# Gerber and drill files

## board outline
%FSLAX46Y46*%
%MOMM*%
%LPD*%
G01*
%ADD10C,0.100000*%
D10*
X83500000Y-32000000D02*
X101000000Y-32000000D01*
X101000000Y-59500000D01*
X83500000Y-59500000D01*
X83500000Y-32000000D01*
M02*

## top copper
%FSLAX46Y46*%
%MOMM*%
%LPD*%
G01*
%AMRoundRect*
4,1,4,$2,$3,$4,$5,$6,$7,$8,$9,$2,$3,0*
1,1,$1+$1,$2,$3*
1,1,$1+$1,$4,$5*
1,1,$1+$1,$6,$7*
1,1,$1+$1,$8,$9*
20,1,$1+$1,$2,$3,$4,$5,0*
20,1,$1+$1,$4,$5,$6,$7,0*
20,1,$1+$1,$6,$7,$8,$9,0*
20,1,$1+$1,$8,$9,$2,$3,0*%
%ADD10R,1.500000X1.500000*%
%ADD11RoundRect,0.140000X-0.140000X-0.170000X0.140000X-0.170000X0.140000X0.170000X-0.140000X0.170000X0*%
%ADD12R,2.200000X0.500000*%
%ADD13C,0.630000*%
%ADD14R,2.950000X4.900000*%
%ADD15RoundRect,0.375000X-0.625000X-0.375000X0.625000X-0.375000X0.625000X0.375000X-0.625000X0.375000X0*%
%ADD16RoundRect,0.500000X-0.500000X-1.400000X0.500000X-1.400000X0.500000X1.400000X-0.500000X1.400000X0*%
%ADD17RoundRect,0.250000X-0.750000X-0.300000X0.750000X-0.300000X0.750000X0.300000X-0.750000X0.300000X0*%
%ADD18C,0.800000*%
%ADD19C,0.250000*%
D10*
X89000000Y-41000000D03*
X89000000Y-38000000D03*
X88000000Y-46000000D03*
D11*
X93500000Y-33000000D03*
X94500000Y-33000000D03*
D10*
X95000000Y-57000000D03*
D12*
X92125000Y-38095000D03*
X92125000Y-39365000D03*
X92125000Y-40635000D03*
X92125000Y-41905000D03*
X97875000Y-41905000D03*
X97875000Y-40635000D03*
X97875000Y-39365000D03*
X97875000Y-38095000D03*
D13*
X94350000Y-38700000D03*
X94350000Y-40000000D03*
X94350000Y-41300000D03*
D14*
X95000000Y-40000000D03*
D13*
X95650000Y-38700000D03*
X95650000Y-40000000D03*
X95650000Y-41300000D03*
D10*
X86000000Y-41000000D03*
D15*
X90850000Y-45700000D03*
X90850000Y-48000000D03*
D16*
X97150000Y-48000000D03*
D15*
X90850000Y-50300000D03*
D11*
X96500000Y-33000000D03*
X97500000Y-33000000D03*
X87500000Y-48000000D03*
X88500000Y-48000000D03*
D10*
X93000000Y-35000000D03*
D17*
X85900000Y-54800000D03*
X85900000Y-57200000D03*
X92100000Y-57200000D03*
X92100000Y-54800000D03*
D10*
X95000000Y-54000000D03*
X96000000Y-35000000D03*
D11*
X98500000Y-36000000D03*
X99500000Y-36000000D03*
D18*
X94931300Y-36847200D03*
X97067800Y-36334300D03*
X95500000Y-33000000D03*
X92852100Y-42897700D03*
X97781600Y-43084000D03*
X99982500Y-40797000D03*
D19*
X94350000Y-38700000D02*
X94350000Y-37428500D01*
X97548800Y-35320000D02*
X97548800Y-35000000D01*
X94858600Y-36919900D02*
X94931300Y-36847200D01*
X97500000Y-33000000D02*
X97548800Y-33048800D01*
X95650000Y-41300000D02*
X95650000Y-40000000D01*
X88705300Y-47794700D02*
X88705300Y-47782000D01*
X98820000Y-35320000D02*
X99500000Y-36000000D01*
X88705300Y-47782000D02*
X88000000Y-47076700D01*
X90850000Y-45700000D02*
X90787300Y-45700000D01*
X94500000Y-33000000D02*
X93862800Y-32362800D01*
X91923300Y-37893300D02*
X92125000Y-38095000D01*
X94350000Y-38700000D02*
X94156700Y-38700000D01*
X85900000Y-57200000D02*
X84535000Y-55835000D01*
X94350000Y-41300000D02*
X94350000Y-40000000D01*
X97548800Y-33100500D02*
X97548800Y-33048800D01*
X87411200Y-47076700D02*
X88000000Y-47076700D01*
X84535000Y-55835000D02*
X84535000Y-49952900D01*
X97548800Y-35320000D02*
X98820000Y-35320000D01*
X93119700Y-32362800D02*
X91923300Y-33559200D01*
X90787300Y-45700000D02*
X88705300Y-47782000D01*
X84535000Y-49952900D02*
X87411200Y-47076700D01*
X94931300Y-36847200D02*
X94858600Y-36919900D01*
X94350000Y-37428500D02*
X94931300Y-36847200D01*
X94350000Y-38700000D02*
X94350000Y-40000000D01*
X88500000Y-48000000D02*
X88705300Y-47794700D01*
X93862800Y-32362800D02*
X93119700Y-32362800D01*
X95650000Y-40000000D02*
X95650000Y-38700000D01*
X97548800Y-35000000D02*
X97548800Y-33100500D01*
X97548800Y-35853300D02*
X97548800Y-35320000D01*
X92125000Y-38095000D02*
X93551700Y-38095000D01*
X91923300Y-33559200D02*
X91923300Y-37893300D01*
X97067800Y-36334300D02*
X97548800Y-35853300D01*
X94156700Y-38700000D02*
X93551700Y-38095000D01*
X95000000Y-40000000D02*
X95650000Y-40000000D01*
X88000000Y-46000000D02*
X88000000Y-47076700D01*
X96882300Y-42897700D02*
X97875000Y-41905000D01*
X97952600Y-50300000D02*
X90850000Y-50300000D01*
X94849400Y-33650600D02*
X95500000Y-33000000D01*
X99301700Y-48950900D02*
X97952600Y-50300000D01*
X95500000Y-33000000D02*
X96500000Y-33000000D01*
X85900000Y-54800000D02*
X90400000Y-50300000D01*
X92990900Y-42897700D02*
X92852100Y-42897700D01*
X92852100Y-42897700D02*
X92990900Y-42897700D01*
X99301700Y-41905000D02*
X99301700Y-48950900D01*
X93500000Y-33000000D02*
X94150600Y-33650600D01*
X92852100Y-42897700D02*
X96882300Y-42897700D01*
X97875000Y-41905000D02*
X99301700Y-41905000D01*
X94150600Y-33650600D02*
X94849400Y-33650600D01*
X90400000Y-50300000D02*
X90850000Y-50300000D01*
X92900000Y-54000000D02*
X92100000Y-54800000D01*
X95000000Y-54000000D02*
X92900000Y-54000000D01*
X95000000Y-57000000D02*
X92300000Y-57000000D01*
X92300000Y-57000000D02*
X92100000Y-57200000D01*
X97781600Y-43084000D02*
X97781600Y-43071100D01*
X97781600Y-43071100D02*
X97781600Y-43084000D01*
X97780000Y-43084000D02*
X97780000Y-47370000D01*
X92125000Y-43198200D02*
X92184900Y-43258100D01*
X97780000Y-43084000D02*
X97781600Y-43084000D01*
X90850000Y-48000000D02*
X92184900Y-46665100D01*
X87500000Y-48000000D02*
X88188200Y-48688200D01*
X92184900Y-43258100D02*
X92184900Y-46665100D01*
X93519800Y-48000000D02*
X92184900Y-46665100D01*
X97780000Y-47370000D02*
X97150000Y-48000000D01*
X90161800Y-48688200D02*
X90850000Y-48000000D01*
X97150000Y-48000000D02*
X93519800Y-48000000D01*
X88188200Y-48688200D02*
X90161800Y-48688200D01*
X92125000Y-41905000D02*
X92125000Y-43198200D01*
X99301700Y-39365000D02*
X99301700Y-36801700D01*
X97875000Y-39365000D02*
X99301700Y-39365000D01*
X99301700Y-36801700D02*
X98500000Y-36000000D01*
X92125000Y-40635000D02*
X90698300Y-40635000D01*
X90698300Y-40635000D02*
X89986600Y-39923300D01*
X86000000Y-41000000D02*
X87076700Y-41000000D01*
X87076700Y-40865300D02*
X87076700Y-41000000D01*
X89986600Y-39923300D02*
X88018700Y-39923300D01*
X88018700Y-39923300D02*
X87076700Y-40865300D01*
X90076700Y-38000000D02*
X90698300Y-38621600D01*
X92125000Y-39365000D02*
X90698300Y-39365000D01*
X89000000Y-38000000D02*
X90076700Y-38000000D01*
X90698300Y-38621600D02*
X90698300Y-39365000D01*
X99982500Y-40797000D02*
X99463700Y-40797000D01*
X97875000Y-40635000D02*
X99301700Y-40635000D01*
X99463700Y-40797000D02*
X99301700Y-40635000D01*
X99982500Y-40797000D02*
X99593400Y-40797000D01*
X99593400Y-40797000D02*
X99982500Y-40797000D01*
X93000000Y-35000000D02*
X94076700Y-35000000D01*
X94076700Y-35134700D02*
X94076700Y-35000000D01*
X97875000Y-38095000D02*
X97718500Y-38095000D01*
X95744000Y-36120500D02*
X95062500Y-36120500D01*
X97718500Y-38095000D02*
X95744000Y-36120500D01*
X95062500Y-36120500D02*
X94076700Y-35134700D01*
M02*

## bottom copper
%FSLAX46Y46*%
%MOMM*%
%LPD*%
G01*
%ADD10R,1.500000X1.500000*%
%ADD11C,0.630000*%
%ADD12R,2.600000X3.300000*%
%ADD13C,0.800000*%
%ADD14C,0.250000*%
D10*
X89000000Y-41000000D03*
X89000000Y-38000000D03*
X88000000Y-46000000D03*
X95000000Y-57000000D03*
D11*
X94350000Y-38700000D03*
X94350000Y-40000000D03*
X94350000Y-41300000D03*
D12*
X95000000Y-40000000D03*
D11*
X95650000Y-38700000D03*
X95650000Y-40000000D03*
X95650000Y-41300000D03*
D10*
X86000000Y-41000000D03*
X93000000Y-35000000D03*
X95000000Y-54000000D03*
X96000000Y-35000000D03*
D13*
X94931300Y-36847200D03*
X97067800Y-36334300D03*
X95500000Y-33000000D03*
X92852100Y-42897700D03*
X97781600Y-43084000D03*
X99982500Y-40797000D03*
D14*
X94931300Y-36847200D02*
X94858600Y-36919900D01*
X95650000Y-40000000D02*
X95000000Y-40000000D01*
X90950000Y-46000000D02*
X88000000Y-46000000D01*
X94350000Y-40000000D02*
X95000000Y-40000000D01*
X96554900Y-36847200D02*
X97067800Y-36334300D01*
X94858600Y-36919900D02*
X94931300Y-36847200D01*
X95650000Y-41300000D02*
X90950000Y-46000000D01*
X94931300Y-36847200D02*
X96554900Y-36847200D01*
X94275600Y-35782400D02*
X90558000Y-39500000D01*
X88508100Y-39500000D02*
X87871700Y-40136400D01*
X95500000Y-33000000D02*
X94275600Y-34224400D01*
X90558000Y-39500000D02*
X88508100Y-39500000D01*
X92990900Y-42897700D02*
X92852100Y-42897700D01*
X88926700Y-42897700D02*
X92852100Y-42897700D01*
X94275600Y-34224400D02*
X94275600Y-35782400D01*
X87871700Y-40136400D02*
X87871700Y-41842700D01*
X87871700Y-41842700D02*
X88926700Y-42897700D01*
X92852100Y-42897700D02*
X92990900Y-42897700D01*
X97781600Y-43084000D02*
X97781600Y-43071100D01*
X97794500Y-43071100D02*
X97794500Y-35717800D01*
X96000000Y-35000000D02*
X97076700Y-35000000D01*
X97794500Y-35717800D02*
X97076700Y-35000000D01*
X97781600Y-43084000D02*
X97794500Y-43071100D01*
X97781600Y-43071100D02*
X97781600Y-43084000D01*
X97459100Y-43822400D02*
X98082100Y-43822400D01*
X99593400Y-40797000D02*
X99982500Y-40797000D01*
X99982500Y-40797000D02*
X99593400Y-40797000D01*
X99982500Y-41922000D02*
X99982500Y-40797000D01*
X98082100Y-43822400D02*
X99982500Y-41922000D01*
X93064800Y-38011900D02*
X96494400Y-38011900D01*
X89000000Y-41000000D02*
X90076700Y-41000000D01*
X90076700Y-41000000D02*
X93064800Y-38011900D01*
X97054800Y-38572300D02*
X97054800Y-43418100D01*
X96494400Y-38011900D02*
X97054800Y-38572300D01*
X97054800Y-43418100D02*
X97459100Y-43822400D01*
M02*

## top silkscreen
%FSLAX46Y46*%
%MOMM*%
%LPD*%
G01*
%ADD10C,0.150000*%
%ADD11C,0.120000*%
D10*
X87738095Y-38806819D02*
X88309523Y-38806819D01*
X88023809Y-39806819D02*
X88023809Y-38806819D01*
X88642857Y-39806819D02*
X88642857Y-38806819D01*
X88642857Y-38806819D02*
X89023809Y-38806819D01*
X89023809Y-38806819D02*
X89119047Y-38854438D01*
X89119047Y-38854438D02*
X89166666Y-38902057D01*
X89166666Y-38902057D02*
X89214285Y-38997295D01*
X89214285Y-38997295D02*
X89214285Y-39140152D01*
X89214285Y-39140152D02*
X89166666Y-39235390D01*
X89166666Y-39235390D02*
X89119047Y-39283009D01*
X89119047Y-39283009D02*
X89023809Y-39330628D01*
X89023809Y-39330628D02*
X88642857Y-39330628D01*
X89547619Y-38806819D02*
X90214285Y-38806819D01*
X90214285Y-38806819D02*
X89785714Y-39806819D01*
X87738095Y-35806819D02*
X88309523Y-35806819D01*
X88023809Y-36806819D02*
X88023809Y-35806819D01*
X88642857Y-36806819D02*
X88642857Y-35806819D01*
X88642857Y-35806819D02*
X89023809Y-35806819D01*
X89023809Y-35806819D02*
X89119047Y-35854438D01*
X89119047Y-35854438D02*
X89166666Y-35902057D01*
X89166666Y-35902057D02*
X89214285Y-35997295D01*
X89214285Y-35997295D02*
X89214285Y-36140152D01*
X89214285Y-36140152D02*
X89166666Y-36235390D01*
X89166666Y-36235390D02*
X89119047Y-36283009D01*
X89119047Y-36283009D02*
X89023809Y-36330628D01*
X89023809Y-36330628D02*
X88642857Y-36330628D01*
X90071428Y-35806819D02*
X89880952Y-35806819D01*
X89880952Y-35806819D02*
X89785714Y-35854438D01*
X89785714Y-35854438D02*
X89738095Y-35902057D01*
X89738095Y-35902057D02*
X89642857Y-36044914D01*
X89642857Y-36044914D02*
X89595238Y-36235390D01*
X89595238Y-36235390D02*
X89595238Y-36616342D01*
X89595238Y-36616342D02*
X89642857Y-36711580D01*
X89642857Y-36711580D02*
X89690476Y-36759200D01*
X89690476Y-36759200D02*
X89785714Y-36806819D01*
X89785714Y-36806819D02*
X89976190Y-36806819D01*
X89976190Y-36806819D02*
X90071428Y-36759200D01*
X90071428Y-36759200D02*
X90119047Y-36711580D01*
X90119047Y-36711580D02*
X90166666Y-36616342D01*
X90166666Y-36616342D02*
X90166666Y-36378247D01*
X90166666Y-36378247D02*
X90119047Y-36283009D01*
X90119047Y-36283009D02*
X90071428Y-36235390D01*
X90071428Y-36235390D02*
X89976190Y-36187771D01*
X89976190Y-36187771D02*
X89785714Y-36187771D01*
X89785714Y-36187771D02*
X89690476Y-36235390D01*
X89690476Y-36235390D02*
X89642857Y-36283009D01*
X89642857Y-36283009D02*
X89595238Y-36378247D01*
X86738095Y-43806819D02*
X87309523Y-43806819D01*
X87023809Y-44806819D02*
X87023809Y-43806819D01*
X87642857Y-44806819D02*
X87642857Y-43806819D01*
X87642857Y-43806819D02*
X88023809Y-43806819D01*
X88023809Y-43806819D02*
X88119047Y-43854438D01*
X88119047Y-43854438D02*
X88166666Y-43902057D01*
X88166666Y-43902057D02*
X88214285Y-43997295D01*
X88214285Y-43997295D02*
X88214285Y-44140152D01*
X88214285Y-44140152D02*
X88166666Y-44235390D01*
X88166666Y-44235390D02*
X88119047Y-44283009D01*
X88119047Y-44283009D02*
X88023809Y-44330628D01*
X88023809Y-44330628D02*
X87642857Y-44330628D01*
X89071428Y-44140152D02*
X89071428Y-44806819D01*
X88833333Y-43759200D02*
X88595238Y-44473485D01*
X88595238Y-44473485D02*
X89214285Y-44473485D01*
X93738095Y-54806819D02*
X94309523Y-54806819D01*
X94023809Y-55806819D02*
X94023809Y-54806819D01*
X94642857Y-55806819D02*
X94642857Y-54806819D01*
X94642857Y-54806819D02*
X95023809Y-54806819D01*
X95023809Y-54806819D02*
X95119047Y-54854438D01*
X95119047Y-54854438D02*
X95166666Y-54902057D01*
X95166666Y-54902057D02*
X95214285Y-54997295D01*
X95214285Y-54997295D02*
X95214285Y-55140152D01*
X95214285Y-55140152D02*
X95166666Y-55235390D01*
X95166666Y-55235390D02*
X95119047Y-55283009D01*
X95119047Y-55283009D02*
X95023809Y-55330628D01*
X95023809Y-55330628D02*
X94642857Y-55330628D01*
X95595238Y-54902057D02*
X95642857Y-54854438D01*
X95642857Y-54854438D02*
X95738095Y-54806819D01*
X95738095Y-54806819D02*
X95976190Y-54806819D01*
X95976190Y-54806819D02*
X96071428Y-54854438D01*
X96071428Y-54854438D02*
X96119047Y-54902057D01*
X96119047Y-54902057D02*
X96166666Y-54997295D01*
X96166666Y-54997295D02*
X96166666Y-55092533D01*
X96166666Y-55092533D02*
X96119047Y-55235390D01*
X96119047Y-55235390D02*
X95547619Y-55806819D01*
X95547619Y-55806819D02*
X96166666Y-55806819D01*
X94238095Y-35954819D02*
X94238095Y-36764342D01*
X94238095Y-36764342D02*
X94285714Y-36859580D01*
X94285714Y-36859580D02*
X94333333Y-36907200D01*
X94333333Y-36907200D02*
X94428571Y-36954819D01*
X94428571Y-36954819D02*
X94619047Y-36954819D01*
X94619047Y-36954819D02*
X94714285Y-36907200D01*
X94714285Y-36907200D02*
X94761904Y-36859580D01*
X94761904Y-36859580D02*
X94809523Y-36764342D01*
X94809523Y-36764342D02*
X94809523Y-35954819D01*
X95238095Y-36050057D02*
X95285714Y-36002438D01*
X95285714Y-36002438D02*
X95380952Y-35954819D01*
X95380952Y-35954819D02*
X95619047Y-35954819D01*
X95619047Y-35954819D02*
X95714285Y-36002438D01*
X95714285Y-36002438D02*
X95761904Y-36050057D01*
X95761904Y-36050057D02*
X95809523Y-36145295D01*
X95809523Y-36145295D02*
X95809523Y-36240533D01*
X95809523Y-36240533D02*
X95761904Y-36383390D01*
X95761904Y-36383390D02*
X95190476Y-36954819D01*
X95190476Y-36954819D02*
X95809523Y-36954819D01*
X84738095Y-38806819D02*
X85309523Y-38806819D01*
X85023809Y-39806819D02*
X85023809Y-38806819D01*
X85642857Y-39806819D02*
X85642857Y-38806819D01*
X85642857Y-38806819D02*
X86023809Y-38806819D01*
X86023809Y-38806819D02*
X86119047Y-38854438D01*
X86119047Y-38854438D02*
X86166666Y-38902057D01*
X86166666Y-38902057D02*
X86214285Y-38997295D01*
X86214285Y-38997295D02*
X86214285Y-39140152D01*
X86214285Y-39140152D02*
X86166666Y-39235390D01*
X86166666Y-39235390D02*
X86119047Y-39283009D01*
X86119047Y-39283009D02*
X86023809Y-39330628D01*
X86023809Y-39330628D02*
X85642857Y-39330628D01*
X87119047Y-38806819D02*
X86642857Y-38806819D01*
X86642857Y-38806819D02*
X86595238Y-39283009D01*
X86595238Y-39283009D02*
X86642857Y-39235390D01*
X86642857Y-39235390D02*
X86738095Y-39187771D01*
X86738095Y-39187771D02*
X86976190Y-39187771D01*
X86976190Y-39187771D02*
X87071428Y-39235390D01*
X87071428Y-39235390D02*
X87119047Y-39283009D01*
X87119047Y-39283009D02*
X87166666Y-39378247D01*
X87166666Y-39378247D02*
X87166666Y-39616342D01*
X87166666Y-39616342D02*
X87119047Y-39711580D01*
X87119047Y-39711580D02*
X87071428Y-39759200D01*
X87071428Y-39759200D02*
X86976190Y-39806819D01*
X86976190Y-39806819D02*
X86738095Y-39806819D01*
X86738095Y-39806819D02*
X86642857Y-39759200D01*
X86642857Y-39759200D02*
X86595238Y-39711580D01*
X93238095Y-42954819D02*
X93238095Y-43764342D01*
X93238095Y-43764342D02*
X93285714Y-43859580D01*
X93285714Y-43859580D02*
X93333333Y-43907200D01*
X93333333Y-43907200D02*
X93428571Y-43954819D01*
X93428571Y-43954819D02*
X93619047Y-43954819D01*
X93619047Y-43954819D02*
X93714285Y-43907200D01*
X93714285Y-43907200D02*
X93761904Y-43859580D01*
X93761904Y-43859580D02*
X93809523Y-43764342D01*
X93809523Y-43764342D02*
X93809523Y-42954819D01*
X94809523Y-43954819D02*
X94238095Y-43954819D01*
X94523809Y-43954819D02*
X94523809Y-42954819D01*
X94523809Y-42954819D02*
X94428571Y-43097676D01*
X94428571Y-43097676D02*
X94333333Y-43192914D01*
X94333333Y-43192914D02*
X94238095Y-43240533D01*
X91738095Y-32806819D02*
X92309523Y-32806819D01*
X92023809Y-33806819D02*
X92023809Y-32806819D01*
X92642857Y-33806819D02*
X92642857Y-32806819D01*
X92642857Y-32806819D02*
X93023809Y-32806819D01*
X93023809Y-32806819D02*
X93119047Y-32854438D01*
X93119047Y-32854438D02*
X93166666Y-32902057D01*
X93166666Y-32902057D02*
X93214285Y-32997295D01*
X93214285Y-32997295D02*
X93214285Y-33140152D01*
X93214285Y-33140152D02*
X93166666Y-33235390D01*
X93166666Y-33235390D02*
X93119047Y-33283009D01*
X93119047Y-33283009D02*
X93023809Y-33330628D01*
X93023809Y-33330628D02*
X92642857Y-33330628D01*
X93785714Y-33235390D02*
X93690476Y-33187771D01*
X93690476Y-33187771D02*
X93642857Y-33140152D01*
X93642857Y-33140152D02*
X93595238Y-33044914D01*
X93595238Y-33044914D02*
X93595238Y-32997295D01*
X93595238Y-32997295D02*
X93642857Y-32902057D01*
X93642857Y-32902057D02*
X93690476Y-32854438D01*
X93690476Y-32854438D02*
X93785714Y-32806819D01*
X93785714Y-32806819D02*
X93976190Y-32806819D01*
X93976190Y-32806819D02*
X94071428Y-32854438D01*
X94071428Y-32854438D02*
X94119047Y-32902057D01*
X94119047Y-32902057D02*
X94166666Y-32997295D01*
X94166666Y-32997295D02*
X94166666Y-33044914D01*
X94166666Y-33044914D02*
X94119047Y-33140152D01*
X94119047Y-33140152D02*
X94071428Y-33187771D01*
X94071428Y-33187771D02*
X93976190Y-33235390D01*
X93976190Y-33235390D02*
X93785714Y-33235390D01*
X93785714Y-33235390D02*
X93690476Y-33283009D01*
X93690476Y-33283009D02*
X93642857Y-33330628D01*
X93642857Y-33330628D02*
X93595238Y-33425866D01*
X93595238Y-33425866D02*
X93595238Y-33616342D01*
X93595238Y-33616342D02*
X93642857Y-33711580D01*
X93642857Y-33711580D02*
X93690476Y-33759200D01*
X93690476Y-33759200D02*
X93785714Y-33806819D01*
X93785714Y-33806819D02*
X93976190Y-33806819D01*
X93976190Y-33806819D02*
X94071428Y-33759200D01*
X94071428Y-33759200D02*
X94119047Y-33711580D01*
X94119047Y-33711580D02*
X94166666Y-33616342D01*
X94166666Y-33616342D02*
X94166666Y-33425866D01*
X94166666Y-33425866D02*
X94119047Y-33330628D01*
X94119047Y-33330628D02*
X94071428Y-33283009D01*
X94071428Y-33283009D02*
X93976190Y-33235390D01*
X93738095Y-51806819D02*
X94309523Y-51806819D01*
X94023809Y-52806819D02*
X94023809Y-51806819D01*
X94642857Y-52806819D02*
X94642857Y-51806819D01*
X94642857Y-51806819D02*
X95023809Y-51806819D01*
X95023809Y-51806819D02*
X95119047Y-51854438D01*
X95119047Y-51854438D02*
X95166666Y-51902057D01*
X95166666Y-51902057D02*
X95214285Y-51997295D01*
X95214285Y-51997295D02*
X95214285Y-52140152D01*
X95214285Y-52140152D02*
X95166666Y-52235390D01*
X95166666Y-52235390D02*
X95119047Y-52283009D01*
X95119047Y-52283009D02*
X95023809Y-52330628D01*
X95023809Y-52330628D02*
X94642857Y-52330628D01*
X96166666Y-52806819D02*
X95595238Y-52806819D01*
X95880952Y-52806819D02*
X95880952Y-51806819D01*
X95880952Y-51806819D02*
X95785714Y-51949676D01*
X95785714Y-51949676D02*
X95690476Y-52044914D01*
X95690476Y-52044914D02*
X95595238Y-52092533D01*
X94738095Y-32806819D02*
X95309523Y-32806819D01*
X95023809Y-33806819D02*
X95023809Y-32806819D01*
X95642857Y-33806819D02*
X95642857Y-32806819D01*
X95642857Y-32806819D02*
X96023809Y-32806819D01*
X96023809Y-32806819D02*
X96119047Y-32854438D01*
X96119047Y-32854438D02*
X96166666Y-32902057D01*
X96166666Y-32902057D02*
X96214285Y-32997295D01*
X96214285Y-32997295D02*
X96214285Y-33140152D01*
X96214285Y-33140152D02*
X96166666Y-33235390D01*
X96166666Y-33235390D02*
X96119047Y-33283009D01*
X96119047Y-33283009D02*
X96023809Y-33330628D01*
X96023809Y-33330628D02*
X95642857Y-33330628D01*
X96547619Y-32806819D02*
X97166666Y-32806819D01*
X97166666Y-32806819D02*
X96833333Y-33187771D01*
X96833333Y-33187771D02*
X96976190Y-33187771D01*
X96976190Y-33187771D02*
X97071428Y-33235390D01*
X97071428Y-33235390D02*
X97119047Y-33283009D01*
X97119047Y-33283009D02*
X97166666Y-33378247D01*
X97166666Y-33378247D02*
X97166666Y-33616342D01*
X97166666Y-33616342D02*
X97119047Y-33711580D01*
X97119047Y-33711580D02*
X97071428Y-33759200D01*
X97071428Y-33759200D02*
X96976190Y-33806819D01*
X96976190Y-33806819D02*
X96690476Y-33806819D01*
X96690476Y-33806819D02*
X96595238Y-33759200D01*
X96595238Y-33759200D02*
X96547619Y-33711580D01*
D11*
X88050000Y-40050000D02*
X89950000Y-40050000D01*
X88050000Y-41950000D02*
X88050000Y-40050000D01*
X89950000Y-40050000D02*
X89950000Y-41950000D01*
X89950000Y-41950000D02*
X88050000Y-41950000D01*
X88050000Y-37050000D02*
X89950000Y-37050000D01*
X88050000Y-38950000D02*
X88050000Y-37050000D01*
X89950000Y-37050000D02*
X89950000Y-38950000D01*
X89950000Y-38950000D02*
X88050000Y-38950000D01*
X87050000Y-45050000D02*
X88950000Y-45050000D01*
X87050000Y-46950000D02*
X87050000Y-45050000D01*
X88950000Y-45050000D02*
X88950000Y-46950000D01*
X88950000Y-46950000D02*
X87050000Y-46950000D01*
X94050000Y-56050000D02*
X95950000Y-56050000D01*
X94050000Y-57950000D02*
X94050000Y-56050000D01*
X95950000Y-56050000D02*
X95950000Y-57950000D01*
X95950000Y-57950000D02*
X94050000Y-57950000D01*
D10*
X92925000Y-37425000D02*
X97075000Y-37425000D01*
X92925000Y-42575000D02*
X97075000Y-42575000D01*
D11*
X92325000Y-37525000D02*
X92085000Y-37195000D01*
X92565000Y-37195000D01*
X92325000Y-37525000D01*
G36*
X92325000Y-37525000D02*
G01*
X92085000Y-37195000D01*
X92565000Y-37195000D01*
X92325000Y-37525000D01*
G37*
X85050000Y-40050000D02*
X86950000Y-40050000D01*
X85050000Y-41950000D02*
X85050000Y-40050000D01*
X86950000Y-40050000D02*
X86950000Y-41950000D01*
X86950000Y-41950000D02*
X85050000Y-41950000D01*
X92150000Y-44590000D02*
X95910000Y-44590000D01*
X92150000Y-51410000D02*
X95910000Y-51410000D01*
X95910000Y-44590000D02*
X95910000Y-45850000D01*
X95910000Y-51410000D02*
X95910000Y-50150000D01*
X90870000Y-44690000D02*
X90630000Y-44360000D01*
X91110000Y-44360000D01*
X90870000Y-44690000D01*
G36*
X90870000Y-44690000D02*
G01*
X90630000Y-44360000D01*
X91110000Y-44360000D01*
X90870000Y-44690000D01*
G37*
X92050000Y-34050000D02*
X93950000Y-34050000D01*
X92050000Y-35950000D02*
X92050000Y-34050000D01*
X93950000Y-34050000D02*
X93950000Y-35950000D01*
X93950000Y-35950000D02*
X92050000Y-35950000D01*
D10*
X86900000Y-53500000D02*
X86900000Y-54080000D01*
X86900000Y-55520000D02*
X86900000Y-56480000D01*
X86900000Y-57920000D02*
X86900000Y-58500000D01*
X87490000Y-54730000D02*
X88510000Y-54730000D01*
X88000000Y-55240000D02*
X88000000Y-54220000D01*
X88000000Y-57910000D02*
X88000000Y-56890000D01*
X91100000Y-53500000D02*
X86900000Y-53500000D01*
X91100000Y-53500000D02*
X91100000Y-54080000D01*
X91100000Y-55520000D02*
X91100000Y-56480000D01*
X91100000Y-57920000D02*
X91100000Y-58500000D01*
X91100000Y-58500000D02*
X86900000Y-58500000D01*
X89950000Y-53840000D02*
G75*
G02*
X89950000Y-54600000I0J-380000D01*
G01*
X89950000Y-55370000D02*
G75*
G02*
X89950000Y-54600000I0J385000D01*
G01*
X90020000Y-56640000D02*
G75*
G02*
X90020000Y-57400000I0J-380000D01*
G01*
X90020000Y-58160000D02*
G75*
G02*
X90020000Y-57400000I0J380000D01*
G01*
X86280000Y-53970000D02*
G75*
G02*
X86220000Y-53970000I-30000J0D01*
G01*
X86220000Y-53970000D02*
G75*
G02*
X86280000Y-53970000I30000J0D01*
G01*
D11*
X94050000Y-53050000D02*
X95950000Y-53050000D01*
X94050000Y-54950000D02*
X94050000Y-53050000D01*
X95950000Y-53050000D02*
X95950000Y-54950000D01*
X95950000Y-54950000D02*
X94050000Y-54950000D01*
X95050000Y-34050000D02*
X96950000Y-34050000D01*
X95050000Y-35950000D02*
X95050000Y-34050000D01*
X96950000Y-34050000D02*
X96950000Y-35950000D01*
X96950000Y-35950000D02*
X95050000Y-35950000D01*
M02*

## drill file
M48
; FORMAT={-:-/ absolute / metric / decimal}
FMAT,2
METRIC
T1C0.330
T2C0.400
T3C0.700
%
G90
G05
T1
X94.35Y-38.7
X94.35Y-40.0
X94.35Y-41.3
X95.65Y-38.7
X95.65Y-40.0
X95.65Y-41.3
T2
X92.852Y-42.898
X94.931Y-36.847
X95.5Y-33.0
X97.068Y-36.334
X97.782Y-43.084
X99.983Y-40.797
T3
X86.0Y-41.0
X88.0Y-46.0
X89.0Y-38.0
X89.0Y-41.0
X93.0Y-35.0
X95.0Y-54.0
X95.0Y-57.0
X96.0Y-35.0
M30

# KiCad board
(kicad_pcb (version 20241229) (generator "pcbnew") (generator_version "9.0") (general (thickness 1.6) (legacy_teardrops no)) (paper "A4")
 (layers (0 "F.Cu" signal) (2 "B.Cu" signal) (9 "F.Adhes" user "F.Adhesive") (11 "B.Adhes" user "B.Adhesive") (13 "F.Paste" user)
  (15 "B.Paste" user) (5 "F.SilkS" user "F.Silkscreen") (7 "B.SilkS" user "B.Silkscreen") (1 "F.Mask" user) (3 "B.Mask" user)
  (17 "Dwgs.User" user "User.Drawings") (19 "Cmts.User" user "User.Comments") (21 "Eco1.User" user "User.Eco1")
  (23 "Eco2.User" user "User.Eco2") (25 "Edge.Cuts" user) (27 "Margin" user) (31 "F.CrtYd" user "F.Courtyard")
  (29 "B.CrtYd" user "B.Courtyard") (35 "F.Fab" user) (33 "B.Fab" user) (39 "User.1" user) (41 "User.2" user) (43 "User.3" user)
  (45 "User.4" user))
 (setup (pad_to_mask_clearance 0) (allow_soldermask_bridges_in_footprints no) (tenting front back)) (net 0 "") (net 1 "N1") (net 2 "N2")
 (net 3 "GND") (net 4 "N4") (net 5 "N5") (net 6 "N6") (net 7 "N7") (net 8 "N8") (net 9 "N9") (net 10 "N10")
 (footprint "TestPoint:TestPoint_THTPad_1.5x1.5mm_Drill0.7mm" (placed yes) (layer "F.Cu") (at 89 41)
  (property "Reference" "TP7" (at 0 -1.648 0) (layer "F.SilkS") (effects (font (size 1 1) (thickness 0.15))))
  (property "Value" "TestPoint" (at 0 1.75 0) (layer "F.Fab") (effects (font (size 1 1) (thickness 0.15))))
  (fp_line (start -0.95 -0.95) (end 0.95 -0.95) (stroke (width 0.12) (type solid)) (layer "F.SilkS"))
  (fp_line (start -0.95 0.95) (end -0.95 -0.95) (stroke (width 0.12) (type solid)) (layer "F.SilkS"))
  (fp_line (start 0.95 -0.95) (end 0.95 0.95) (stroke (width 0.12) (type solid)) (layer "F.SilkS"))
  (fp_line (start 0.95 0.95) (end -0.95 0.95) (stroke (width 0.12) (type solid)) (layer "F.SilkS"))
  (pad "1" thru_hole rect (at 0 0) (size 1.5 1.5) (drill 0.7) (layers "*.Cu" "*.Mask") (remove_unused_layers no) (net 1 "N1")))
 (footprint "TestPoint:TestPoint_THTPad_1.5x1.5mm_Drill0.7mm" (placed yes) (layer "F.Cu") (at 89 38)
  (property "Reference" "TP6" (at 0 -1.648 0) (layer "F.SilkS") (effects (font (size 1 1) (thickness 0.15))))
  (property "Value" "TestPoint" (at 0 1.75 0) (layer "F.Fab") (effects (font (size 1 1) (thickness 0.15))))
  (fp_line (start -0.95 -0.95) (end 0.95 -0.95) (stroke (width 0.12) (type solid)) (layer "F.SilkS"))
  (fp_line (start -0.95 0.95) (end -0.95 -0.95) (stroke (width 0.12) (type solid)) (layer "F.SilkS"))
  (fp_line (start 0.95 -0.95) (end 0.95 0.95) (stroke (width 0.12) (type solid)) (layer "F.SilkS"))
  (fp_line (start 0.95 0.95) (end -0.95 0.95) (stroke (width 0.12) (type solid)) (layer "F.SilkS"))
  (pad "1" thru_hole rect (at 0 0) (size 1.5 1.5) (drill 0.7) (layers "*.Cu" "*.Mask") (remove_unused_layers no) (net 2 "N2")))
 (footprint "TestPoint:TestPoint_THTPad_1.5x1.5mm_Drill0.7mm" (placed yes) (layer "F.Cu") (at 88 46)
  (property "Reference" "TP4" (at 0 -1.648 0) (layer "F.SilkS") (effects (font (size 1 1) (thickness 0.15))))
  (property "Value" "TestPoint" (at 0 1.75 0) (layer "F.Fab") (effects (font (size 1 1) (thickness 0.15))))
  (fp_line (start -0.95 -0.95) (end 0.95 -0.95) (stroke (width 0.12) (type solid)) (layer "F.SilkS"))
  (fp_line (start -0.95 0.95) (end -0.95 -0.95) (stroke (width 0.12) (type solid)) (layer "F.SilkS"))
  (fp_line (start 0.95 -0.95) (end 0.95 0.95) (stroke (width 0.12) (type solid)) (layer "F.SilkS"))
  (fp_line (start 0.95 0.95) (end -0.95 0.95) (stroke (width 0.12) (type solid)) (layer "F.SilkS"))
  (pad "1" thru_hole rect (at 0 0) (size 1.5 1.5) (drill 0.7) (layers "*.Cu" "*.Mask") (remove_unused_layers no) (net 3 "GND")))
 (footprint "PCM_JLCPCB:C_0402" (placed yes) (layer "F.Cu") (at 94 33)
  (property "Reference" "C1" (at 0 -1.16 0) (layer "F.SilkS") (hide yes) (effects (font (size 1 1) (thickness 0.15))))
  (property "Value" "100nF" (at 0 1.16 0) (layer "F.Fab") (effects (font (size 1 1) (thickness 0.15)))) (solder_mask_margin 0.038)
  (pad "1" smd roundrect (at -0.5 0) (size 0.56 0.62) (layers "F.Cu" "F.Mask" "F.Paste") (roundrect_rratio 0.25) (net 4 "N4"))
  (pad "2" smd roundrect (at 0.5 0) (size 0.56 0.62) (layers "F.Cu" "F.Mask" "F.Paste") (roundrect_rratio 0.25) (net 3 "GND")))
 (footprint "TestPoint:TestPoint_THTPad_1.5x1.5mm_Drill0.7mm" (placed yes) (layer "F.Cu") (at 95 57)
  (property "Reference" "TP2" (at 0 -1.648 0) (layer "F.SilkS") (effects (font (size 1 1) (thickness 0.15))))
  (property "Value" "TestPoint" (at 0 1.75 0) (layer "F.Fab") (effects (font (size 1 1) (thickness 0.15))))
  (fp_line (start -0.95 -0.95) (end 0.95 -0.95) (stroke (width 0.12) (type solid)) (layer "F.SilkS"))
  (fp_line (start -0.95 0.95) (end -0.95 -0.95) (stroke (width 0.12) (type solid)) (layer "F.SilkS"))
  (fp_line (start 0.95 -0.95) (end 0.95 0.95) (stroke (width 0.12) (type solid)) (layer "F.SilkS"))
  (fp_line (start 0.95 0.95) (end -0.95 0.95) (stroke (width 0.12) (type solid)) (layer "F.SilkS"))
  (pad "1" thru_hole rect (at 0 0) (size 1.5 1.5) (drill 0.7) (layers "*.Cu" "*.Mask") (remove_unused_layers no) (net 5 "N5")))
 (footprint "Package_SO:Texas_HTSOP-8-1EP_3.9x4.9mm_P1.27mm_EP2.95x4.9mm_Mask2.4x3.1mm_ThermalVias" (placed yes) (layer "F.Cu") (at 95 40)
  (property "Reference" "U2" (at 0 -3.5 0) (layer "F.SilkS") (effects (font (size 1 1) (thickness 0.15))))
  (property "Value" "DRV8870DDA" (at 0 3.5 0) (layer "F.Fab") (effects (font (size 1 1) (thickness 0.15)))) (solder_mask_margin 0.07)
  (fp_line (start -2.075 -2.575) (end 2.075 -2.575) (stroke (width 0.15) (type solid)) (layer "F.SilkS"))
  (fp_line (start -2.075 2.575) (end 2.075 2.575) (stroke (width 0.15) (type solid)) (layer "F.SilkS"))
  (fp_poly
   (pts (xy -2.675 -2.475) (xy -2.915 -2.805) (xy -2.435 -2.805) (xy -2.675 -2.475)) (stroke (width 0.12) (type solid)) (fill yes)
   (layer "F.SilkS"))
  (pad "" smd rect (at 0 0) (size 2.4 3.1) (layers "F.Mask")) (pad "" smd rect (at 0 0) (size 2.4 3.1) (layers "F.Paste"))
  (pad "1" smd rect (at -2.875 -1.905) (size 2.2 0.5) (layers "F.Cu" "F.Mask" "F.Paste") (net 3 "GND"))
  (pad "2" smd rect (at -2.875 -0.635) (size 2.2 0.5) (layers "F.Cu" "F.Mask" "F.Paste") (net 2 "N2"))
  (pad "3" smd rect (at -2.875 0.635) (size 2.2 0.5) (layers "F.Cu" "F.Mask" "F.Paste") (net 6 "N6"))
  (pad "4" smd rect (at -2.875 1.905) (size 2.2 0.5) (layers "F.Cu" "F.Mask" "F.Paste") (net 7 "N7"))
  (pad "5" smd rect (at 2.875 1.905) (size 2.2 0.5) (layers "F.Cu" "F.Mask" "F.Paste") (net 4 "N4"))
  (pad "6" smd rect (at 2.875 0.635) (size 2.2 0.5) (layers "F.Cu" "F.Mask" "F.Paste") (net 1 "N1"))
  (pad "7" smd rect (at 2.875 -0.635) (size 2.2 0.5) (layers "F.Cu" "F.Mask" "F.Paste") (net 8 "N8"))
  (pad "8" smd rect (at 2.875 -1.905) (size 2.2 0.5) (layers "F.Cu" "F.Mask" "F.Paste") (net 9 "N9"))
  (pad "9" thru_hole circle (at -0.65 -1.3) (size 0.63 0.63) (drill 0.33) (layers "*.Cu" "*.Mask") (remove_unused_layers no) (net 3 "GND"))
  (pad "9" thru_hole circle (at -0.65 0) (size 0.63 0.63) (drill 0.33) (layers "*.Cu" "*.Mask") (remove_unused_layers no) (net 3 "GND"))
  (pad "9" thru_hole circle (at -0.65 1.3) (size 0.63 0.63) (drill 0.33) (layers "*.Cu" "*.Mask") (remove_unused_layers no) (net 3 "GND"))
  (pad "9" smd rect (at 0 0) (size 2.6 3.3) (layers "B.Cu") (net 3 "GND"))
  (pad "9" smd rect (at 0 0) (size 2.95 4.9) (layers "F.Cu") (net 3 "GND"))
  (pad "9" thru_hole circle (at 0.65 -1.3) (size 0.63 0.63) (drill 0.33) (layers "*.Cu" "*.Mask") (remove_unused_layers no) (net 3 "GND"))
  (pad "9" thru_hole circle (at 0.65 0) (size 0.63 0.63) (drill 0.33) (layers "*.Cu" "*.Mask") (remove_unused_layers no) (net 3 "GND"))
  (pad "9" thru_hole circle (at 0.65 1.3) (size 0.63 0.63) (drill 0.33) (layers "*.Cu" "*.Mask") (remove_unused_layers no) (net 3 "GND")))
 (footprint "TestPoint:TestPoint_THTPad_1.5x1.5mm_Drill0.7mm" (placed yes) (layer "F.Cu") (at 86 41)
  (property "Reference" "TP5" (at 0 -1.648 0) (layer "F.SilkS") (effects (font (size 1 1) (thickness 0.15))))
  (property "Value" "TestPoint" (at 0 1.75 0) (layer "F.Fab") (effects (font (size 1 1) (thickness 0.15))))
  (fp_line (start -0.95 -0.95) (end 0.95 -0.95) (stroke (width 0.12) (type solid)) (layer "F.SilkS"))
  (fp_line (start -0.95 0.95) (end -0.95 -0.95) (stroke (width 0.12) (type solid)) (layer "F.SilkS"))
  (fp_line (start 0.95 -0.95) (end 0.95 0.95) (stroke (width 0.12) (type solid)) (layer "F.SilkS"))
  (fp_line (start 0.95 0.95) (end -0.95 0.95) (stroke (width 0.12) (type solid)) (layer "F.SilkS"))
  (pad "1" thru_hole rect (at 0 0) (size 1.5 1.5) (drill 0.7) (layers "*.Cu" "*.Mask") (remove_unused_layers no) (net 6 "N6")))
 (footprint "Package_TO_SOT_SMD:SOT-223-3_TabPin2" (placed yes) (layer "F.Cu") (at 94 48)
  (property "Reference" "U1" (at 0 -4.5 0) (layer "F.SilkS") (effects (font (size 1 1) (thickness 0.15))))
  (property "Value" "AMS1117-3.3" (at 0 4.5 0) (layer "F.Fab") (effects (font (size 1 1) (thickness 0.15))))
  (fp_line (start -1.85 -3.41) (end 1.91 -3.41) (stroke (width 0.12) (type solid)) (layer "F.SilkS"))
  (fp_line (start -1.85 3.41) (end 1.91 3.41) (stroke (width 0.12) (type solid)) (layer "F.SilkS"))
  (fp_line (start 1.91 -3.41) (end 1.91 -2.15) (stroke (width 0.12) (type solid)) (layer "F.SilkS"))
  (fp_line (start 1.91 3.41) (end 1.91 2.15) (stroke (width 0.12) (type solid)) (layer "F.SilkS"))
  (fp_poly
   (pts (xy -3.13 -3.31) (xy -3.37 -3.64) (xy -2.89 -3.64) (xy -3.13 -3.31)) (stroke (width 0.12) (type solid)) (fill yes) (layer "F.SilkS"))
  (pad "1" smd roundrect (at -3.15 -2.3) (size 2 1.5) (layers "F.Cu" "F.Mask" "F.Paste") (roundrect_rratio 0.25) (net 3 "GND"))
  (pad "2" smd roundrect (at -3.15 0) (size 2 1.5) (layers "F.Cu" "F.Mask" "F.Paste") (roundrect_rratio 0.25) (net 7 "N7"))
  (pad "2" smd roundrect (at 3.15 0) (size 2 3.8) (layers "F.Cu" "F.Mask" "F.Paste") (roundrect_rratio 0.25) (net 7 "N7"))
  (pad "3" smd roundrect (at -3.15 2.3) (size 2 1.5) (layers "F.Cu" "F.Mask" "F.Paste") (roundrect_rratio 0.25) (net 4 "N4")))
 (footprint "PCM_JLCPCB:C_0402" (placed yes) (layer "F.Cu") (at 97 33)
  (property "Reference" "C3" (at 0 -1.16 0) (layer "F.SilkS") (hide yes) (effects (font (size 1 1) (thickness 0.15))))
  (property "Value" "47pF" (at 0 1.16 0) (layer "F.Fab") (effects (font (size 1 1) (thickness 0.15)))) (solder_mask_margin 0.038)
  (pad "1" smd roundrect (at -0.5 0) (size 0.56 0.62) (layers "F.Cu" "F.Mask" "F.Paste") (roundrect_rratio 0.25) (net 4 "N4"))
  (pad "2" smd roundrect (at 0.5 0) (size 0.56 0.62) (layers "F.Cu" "F.Mask" "F.Paste") (roundrect_rratio 0.25) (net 3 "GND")))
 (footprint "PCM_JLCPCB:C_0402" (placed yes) (layer "F.Cu") (at 88 48)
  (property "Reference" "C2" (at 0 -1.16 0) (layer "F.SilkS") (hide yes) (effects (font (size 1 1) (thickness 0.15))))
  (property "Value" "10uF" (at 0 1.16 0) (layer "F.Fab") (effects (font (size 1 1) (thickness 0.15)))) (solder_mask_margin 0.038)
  (pad "1" smd roundrect (at -0.5 0) (size 0.56 0.62) (layers "F.Cu" "F.Mask" "F.Paste") (roundrect_rratio 0.25) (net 7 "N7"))
  (pad "2" smd roundrect (at 0.5 0) (size 0.56 0.62) (layers "F.Cu" "F.Mask" "F.Paste") (roundrect_rratio 0.25) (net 3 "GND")))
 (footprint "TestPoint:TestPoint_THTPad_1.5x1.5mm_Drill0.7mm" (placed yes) (layer "F.Cu") (at 93 35)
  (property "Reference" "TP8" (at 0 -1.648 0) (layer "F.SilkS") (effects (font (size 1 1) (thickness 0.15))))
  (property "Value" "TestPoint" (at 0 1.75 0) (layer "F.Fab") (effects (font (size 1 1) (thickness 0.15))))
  (fp_line (start -0.95 -0.95) (end 0.95 -0.95) (stroke (width 0.12) (type solid)) (layer "F.SilkS"))
  (fp_line (start -0.95 0.95) (end -0.95 -0.95) (stroke (width 0.12) (type solid)) (layer "F.SilkS"))
  (fp_line (start 0.95 -0.95) (end 0.95 0.95) (stroke (width 0.12) (type solid)) (layer "F.SilkS"))
  (fp_line (start 0.95 0.95) (end -0.95 0.95) (stroke (width 0.12) (type solid)) (layer "F.SilkS"))
  (pad "1" thru_hole rect (at 0 0) (size 1.5 1.5) (drill 0.7) (layers "*.Cu" "*.Mask") (remove_unused_layers no) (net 9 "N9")))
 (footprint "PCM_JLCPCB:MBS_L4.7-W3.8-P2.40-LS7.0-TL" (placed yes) (layer "F.Cu") (at 89 56)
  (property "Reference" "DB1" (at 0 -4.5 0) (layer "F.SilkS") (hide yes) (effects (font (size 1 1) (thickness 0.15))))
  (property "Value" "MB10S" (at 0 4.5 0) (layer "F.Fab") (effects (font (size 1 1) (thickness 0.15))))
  (fp_line (start -2.1 -2.5) (end -2.1 -1.92) (stroke (width 0.15) (type solid)) (layer "F.SilkS"))
  (fp_line (start -2.1 -0.48) (end -2.1 0.48) (stroke (width 0.15) (type solid)) (layer "F.SilkS"))
  (fp_line (start -2.1 1.92) (end -2.1 2.5) (stroke (width 0.15) (type solid)) (layer "F.SilkS"))
  (fp_line (start -1.51 -1.27) (end -0.49 -1.27) (stroke (width 0.15) (type solid)) (layer "F.SilkS"))
  (fp_line (start -1 -0.76) (end -1 -1.78) (stroke (width 0.15) (type solid)) (layer "F.SilkS"))
  (fp_line (start -1 1.91) (end -1 0.89) (stroke (width 0.15) (type solid)) (layer "F.SilkS"))
  (fp_line (start 2.1 -2.5) (end -2.1 -2.5) (stroke (width 0.15) (type solid)) (layer "F.SilkS"))
  (fp_line (start 2.1 -2.5) (end 2.1 -1.92) (stroke (width 0.15) (type solid)) (layer "F.SilkS"))
  (fp_line (start 2.1 -0.48) (end 2.1 0.48) (stroke (width 0.15) (type solid)) (layer "F.SilkS"))
  (fp_line (start 2.1 1.92) (end 2.1 2.5) (stroke (width 0.15) (type solid)) (layer "F.SilkS"))
  (fp_line (start 2.1 2.5) (end -2.1 2.5) (stroke (width 0.15) (type solid)) (layer "F.SilkS"))
  (fp_arc (start 0.95 -2.16) (mid 1.33 -1.78) (end 0.95 -1.4) (stroke (width 0.15) (type solid)) (layer "F.SilkS"))
  (fp_arc (start 0.95 -0.63) (mid 0.565 -1.015) (end 0.95 -1.4) (stroke (width 0.15) (type solid)) (layer "F.SilkS"))
  (fp_arc (start 1.02 0.64) (mid 1.4 1.02) (end 1.02 1.4) (stroke (width 0.15) (type solid)) (layer "F.SilkS"))
  (fp_arc (start 1.02 2.16) (mid 0.64 1.78) (end 1.02 1.4) (stroke (width 0.15) (type solid)) (layer "F.SilkS"))
  (fp_circle (center -2.75 -2.03) (end -2.72 -2.03) (stroke (width 0.15) (type solid)) (fill no) (layer "F.SilkS"))
  (pad "1" smd roundrect (at -3.1 -1.2) (size 2 1.1) (layers "F.Cu" "F.Mask" "F.Paste") (roundrect_rratio 0.2272727273) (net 4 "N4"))
  (pad "2" smd roundrect (at -3.1 1.2) (size 2 1.1) (layers "F.Cu" "F.Mask" "F.Paste") (roundrect_rratio 0.2272727273) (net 3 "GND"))
  (pad "3" smd roundrect (at 3.1 1.2) (size 2 1.1) (layers "F.Cu" "F.Mask" "F.Paste") (roundrect_rratio 0.2272727273) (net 5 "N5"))
  (pad "4" smd roundrect (at 3.1 -1.2) (size 2 1.1) (layers "F.Cu" "F.Mask" "F.Paste") (roundrect_rratio 0.2272727273) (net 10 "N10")))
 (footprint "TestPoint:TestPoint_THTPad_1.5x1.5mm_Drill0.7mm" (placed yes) (layer "F.Cu") (at 95 54)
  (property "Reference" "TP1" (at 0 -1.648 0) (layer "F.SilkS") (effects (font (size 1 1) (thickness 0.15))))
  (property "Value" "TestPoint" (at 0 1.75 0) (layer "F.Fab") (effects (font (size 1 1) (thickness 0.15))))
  (fp_line (start -0.95 -0.95) (end 0.95 -0.95) (stroke (width 0.12) (type solid)) (layer "F.SilkS"))
  (fp_line (start -0.95 0.95) (end -0.95 -0.95) (stroke (width 0.12) (type solid)) (layer "F.SilkS"))
  (fp_line (start 0.95 -0.95) (end 0.95 0.95) (stroke (width 0.12) (type solid)) (layer "F.SilkS"))
  (fp_line (start 0.95 0.95) (end -0.95 0.95) (stroke (width 0.12) (type solid)) (layer "F.SilkS"))
  (pad "1" thru_hole rect (at 0 0) (size 1.5 1.5) (drill 0.7) (layers "*.Cu" "*.Mask") (remove_unused_layers no) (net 10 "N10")))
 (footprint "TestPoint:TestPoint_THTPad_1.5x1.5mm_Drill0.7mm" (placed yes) (layer "F.Cu") (at 96 35)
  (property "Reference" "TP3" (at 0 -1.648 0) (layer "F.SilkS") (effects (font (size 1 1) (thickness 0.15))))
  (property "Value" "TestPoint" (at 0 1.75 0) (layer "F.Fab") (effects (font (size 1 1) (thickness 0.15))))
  (fp_line (start -0.95 -0.95) (end 0.95 -0.95) (stroke (width 0.12) (type solid)) (layer "F.SilkS"))
  (fp_line (start -0.95 0.95) (end -0.95 -0.95) (stroke (width 0.12) (type solid)) (layer "F.SilkS"))
  (fp_line (start 0.95 -0.95) (end 0.95 0.95) (stroke (width 0.12) (type solid)) (layer "F.SilkS"))
  (fp_line (start 0.95 0.95) (end -0.95 0.95) (stroke (width 0.12) (type solid)) (layer "F.SilkS"))
  (pad "1" thru_hole rect (at 0 0) (size 1.5 1.5) (drill 0.7) (layers "*.Cu" "*.Mask") (remove_unused_layers no) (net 7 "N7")))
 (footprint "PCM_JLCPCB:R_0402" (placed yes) (layer "F.Cu") (at 99 36)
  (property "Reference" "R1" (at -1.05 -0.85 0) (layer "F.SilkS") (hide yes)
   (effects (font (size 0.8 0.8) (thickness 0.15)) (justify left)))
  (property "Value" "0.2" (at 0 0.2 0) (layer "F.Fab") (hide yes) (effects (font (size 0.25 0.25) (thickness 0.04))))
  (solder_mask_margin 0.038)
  (pad "1" smd roundrect (at -0.5 0) (size 0.56 0.62) (layers "F.Cu" "F.Mask" "F.Paste") (roundrect_rratio 0.25) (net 8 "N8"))
  (pad "2" smd roundrect (at 0.5 0) (size 0.56 0.62) (layers "F.Cu" "F.Mask" "F.Paste") (roundrect_rratio 0.25) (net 3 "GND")))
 (gr_rect (start 83.5 32) (end 101 59.5) (stroke (width 0.1) (type default)) (fill no) (layer "Edge.Cuts"))
 (segment (start 94.35 38.7) (end 94.35 37.4285) (width 0.25) (layer "F.Cu") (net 3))
 (segment (start 97.5488 35.32) (end 97.5488 35) (width 0.25) (layer "F.Cu") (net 3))
 (segment (start 94.8586 36.9199) (end 94.9313 36.8472) (width 0.25) (layer "F.Cu") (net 3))
 (segment (start 97.5 33) (end 97.5488 33.0488) (width 0.25) (layer "F.Cu") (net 3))
 (segment (start 95.65 41.3) (end 95.65 40) (width 0.25) (layer "F.Cu") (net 3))
 (segment (start 88.7053 47.7947) (end 88.7053 47.782) (width 0.25) (layer "F.Cu") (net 3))
 (segment (start 98.82 35.32) (end 99.5 36) (width 0.25) (layer "F.Cu") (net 3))
 (segment (start 88.7053 47.782) (end 88 47.0767) (width 0.25) (layer "F.Cu") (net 3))
 (segment (start 90.85 45.7) (end 90.7873 45.7) (width 0.25) (layer "F.Cu") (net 3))
 (segment (start 94.5 33) (end 93.8628 32.3628) (width 0.25) (layer "F.Cu") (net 3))
 (segment (start 91.9233 37.8933) (end 92.125 38.095) (width 0.25) (layer "F.Cu") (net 3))
 (segment (start 94.35 38.7) (end 94.1567 38.7) (width 0.25) (layer "F.Cu") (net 3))
 (segment (start 85.9 57.2) (end 84.535 55.835) (width 0.25) (layer "F.Cu") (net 3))
 (segment (start 94.35 41.3) (end 94.35 40) (width 0.25) (layer "F.Cu") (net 3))
 (segment (start 97.5488 33.1005) (end 97.5488 33.0488) (width 0.25) (layer "F.Cu") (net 3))
 (segment (start 87.4112 47.0767) (end 88 47.0767) (width 0.25) (layer "F.Cu") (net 3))
 (segment (start 84.535 55.835) (end 84.535 49.9529) (width 0.25) (layer "F.Cu") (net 3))
 (segment (start 97.5488 35.32) (end 98.82 35.32) (width 0.25) (layer "F.Cu") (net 3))
 (segment (start 93.1197 32.3628) (end 91.9233 33.5592) (width 0.25) (layer "F.Cu") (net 3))
 (segment (start 90.7873 45.7) (end 88.7053 47.782) (width 0.25) (layer "F.Cu") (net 3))
 (segment (start 84.535 49.9529) (end 87.4112 47.0767) (width 0.25) (layer "F.Cu") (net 3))
 (segment (start 94.9313 36.8472) (end 94.8586 36.9199) (width 0.25) (layer "F.Cu") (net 3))
 (segment (start 94.35 37.4285) (end 94.9313 36.8472) (width 0.25) (layer "F.Cu") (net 3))
 (segment (start 94.35 38.7) (end 94.35 40) (width 0.25) (layer "F.Cu") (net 3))
 (segment (start 88.5 48) (end 88.7053 47.7947) (width 0.25) (layer "F.Cu") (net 3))
 (segment (start 93.8628 32.3628) (end 93.1197 32.3628) (width 0.25) (layer "F.Cu") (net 3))
 (segment (start 95.65 40) (end 95.65 38.7) (width 0.25) (layer "F.Cu") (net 3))
 (segment (start 97.5488 35) (end 97.5488 33.1005) (width 0.25) (layer "F.Cu") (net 3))
 (segment (start 97.5488 35.8533) (end 97.5488 35.32) (width 0.25) (layer "F.Cu") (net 3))
 (segment (start 92.125 38.095) (end 93.5517 38.095) (width 0.25) (layer "F.Cu") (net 3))
 (segment (start 91.9233 33.5592) (end 91.9233 37.8933) (width 0.25) (layer "F.Cu") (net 3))
 (segment (start 97.0678 36.3343) (end 97.5488 35.8533) (width 0.25) (layer "F.Cu") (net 3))
 (segment (start 94.1567 38.7) (end 93.5517 38.095) (width 0.25) (layer "F.Cu") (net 3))
 (segment (start 95 40) (end 95.65 40) (width 0.25) (layer "F.Cu") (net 3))
 (segment (start 88 46) (end 88 47.0767) (width 0.25) (layer "F.Cu") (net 3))
 (via (at 94.9313 36.8472) (size 0.8) (drill 0.4) (layers "F.Cu" "B.Cu") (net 3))
 (via (at 97.0678 36.3343) (size 0.8) (drill 0.4) (layers "F.Cu" "B.Cu") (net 3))
 (segment (start 94.9313 36.8472) (end 94.8586 36.9199) (width 0.25) (layer "B.Cu") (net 3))
 (segment (start 95.65 40) (end 95 40) (width 0.25) (layer "B.Cu") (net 3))
 (segment (start 90.95 46) (end 88 46) (width 0.25) (layer "B.Cu") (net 3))
 (segment (start 94.35 40) (end 95 40) (width 0.25) (layer "B.Cu") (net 3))
 (segment (start 96.5549 36.8472) (end 97.0678 36.3343) (width 0.25) (layer "B.Cu") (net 3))
 (segment (start 94.8586 36.9199) (end 94.9313 36.8472) (width 0.25) (layer "B.Cu") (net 3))
 (segment (start 95.65 41.3) (end 90.95 46) (width 0.25) (layer "B.Cu") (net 3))
 (segment (start 94.9313 36.8472) (end 96.5549 36.8472) (width 0.25) (layer "B.Cu") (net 3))
 (segment (start 96.8823 42.8977) (end 97.875 41.905) (width 0.25) (layer "F.Cu") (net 4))
 (segment (start 97.9526 50.3) (end 90.85 50.3) (width 0.25) (layer "F.Cu") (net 4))
 (segment (start 94.8494 33.6506) (end 95.5 33) (width 0.25) (layer "F.Cu") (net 4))
 (segment (start 99.3017 48.9509) (end 97.9526 50.3) (width 0.25) (layer "F.Cu") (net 4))
 (segment (start 95.5 33) (end 96.5 33) (width 0.25) (layer "F.Cu") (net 4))
 (segment (start 85.9 54.8) (end 90.4 50.3) (width 0.25) (layer "F.Cu") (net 4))
 (segment (start 92.9909 42.8977) (end 92.8521 42.8977) (width 0.25) (layer "F.Cu") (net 4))
 (segment (start 92.8521 42.8977) (end 92.9909 42.8977) (width 0.25) (layer "F.Cu") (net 4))
 (segment (start 99.3017 41.905) (end 99.3017 48.9509) (width 0.25) (layer "F.Cu") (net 4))
 (segment (start 93.5 33) (end 94.1506 33.6506) (width 0.25) (layer "F.Cu") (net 4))
 (segment (start 92.8521 42.8977) (end 96.8823 42.8977) (width 0.25) (layer "F.Cu") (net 4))
 (segment (start 97.875 41.905) (end 99.3017 41.905) (width 0.25) (layer "F.Cu") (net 4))
 (segment (start 94.1506 33.6506) (end 94.8494 33.6506) (width 0.25) (layer "F.Cu") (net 4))
 (segment (start 90.4 50.3) (end 90.85 50.3) (width 0.25) (layer "F.Cu") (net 4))
 (via (at 95.5 33) (size 0.8) (drill 0.4) (layers "F.Cu" "B.Cu") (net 4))
 (via (at 92.8521 42.8977) (size 0.8) (drill 0.4) (layers "F.Cu" "B.Cu") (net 4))
 (segment (start 94.2756 35.7824) (end 90.558 39.5) (width 0.25) (layer "B.Cu") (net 4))
 (segment (start 88.5081 39.5) (end 87.8717 40.1364) (width 0.25) (layer "B.Cu") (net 4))
 (segment (start 95.5 33) (end 94.2756 34.2244) (width 0.25) (layer "B.Cu") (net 4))
 (segment (start 90.558 39.5) (end 88.5081 39.5) (width 0.25) (layer "B.Cu") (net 4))
 (segment (start 92.9909 42.8977) (end 92.8521 42.8977) (width 0.25) (layer "B.Cu") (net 4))
 (segment (start 88.9267 42.8977) (end 92.8521 42.8977) (width 0.25) (layer "B.Cu") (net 4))
 (segment (start 94.2756 34.2244) (end 94.2756 35.7824) (width 0.25) (layer "B.Cu") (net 4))
 (segment (start 87.8717 40.1364) (end 87.8717 41.8427) (width 0.25) (layer "B.Cu") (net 4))
 (segment (start 87.8717 41.8427) (end 88.9267 42.8977) (width 0.25) (layer "B.Cu") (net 4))
 (segment (start 92.8521 42.8977) (end 92.9909 42.8977) (width 0.25) (layer "B.Cu") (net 4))
 (segment (start 92.9 54) (end 92.1 54.8) (width 0.25) (layer "F.Cu") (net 10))
 (segment (start 95 54) (end 92.9 54) (width 0.25) (layer "F.Cu") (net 10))
 (segment (start 95 57) (end 92.3 57) (width 0.25) (layer "F.Cu") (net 5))
 (segment (start 92.3 57) (end 92.1 57.2) (width 0.25) (layer "F.Cu") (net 5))
 (segment (start 97.7816 43.084) (end 97.7816 43.0711) (width 0.25) (layer "F.Cu") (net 7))
 (segment (start 97.7816 43.0711) (end 97.7816 43.084) (width 0.25) (layer "F.Cu") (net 7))
 (segment (start 97.78 43.084) (end 97.78 47.37) (width 0.25) (layer "F.Cu") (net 7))
 (segment (start 92.125 43.1982) (end 92.1849 43.2581) (width 0.25) (layer "F.Cu") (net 7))
 (segment (start 97.78 43.084) (end 97.7816 43.084) (width 0.25) (layer "F.Cu") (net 7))
 (segment (start 90.85 48) (end 92.1849 46.6651) (width 0.25) (layer "F.Cu") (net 7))
 (segment (start 87.5 48) (end 88.1882 48.6882) (width 0.25) (layer "F.Cu") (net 7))
 (segment (start 92.1849 43.2581) (end 92.1849 46.6651) (width 0.25) (layer "F.Cu") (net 7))
 (segment (start 93.5198 48) (end 92.1849 46.6651) (width 0.25) (layer "F.Cu") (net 7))
 (segment (start 97.78 47.37) (end 97.15 48) (width 0.25) (layer "F.Cu") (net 7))
 (segment (start 90.1618 48.6882) (end 90.85 48) (width 0.25) (layer "F.Cu") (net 7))
 (segment (start 97.15 48) (end 93.5198 48) (width 0.25) (layer "F.Cu") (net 7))
 (segment (start 88.1882 48.6882) (end 90.1618 48.6882) (width 0.25) (layer "F.Cu") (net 7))
 (segment (start 92.125 41.905) (end 92.125 43.1982) (width 0.25) (layer "F.Cu") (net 7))
 (via (at 97.7816 43.084) (size 0.8) (drill 0.4) (layers "F.Cu" "B.Cu") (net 7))
 (segment (start 97.7816 43.084) (end 97.7816 43.0711) (width 0.25) (layer "B.Cu") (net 7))
 (segment (start 97.7945 43.0711) (end 97.7945 35.7178) (width 0.25) (layer "B.Cu") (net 7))
 (segment (start 96 35) (end 97.0767 35) (width 0.25) (layer "B.Cu") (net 7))
 (segment (start 97.7945 35.7178) (end 97.0767 35) (width 0.25) (layer "B.Cu") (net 7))
 (segment (start 97.7816 43.084) (end 97.7945 43.0711) (width 0.25) (layer "B.Cu") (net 7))
 (segment (start 97.7816 43.0711) (end 97.7816 43.084) (width 0.25) (layer "B.Cu") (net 7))
 (segment (start 99.3017 39.365) (end 99.3017 36.8017) (width 0.25) (layer "F.Cu") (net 8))
 (segment (start 97.875 39.365) (end 99.3017 39.365) (width 0.25) (layer "F.Cu") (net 8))
 (segment (start 99.3017 36.8017) (end 98.5 36) (width 0.25) (layer "F.Cu") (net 8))
 (segment (start 92.125 40.635) (end 90.6983 40.635) (width 0.25) (layer "F.Cu") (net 6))
 (segment (start 90.6983 40.635) (end 89.9866 39.9233) (width 0.25) (layer "F.Cu") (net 6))
 (segment (start 86 41) (end 87.0767 41) (width 0.25) (layer "F.Cu") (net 6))
 (segment (start 87.0767 40.8653) (end 87.0767 41) (width 0.25) (layer "F.Cu") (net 6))
 (segment (start 89.9866 39.9233) (end 88.0187 39.9233) (width 0.25) (layer "F.Cu") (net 6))
 (segment (start 88.0187 39.9233) (end 87.0767 40.8653) (width 0.25) (layer "F.Cu") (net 6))
 (segment (start 90.0767 38) (end 90.6983 38.6216) (width 0.25) (layer "F.Cu") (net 2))
 (segment (start 92.125 39.365) (end 90.6983 39.365) (width 0.25) (layer "F.Cu") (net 2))
 (segment (start 89 38) (end 90.0767 38) (width 0.25) (layer "F.Cu") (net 2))
 (segment (start 90.6983 38.6216) (end 90.6983 39.365) (width 0.25) (layer "F.Cu") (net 2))
 (segment (start 99.9825 40.797) (end 99.4637 40.797) (width 0.25) (layer "F.Cu") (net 1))
 (segment (start 97.875 40.635) (end 99.3017 40.635) (width 0.25) (layer "F.Cu") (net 1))
 (segment (start 99.4637 40.797) (end 99.3017 40.635) (width 0.25) (layer "F.Cu") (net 1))
 (segment (start 99.9825 40.797) (end 99.5934 40.797) (width 0.25) (layer "F.Cu") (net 1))
 (segment (start 99.5934 40.797) (end 99.9825 40.797) (width 0.25) (layer "F.Cu") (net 1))
 (via (at 99.9825 40.797) (size 0.8) (drill 0.4) (layers "F.Cu" "B.Cu") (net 1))
 (segment (start 97.4591 43.8224) (end 98.0821 43.8224) (width 0.25) (layer "B.Cu") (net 1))
 (segment (start 99.5934 40.797) (end 99.9825 40.797) (width 0.25) (layer "B.Cu") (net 1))
 (segment (start 99.9825 40.797) (end 99.5934 40.797) (width 0.25) (layer "B.Cu") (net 1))
 (segment (start 99.9825 41.922) (end 99.9825 40.797) (width 0.25) (layer "B.Cu") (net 1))
 (segment (start 98.0821 43.8224) (end 99.9825 41.922) (width 0.25) (layer "B.Cu") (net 1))
 (segment (start 93.0648 38.0119) (end 96.4944 38.0119) (width 0.25) (layer "B.Cu") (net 1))
 (segment (start 89 41) (end 90.0767 41) (width 0.25) (layer "B.Cu") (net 1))
 (segment (start 90.0767 41) (end 93.0648 38.0119) (width 0.25) (layer "B.Cu") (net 1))
 (segment (start 97.0548 38.5723) (end 97.0548 43.4181) (width 0.25) (layer "B.Cu") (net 1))
 (segment (start 96.4944 38.0119) (end 97.0548 38.5723) (width 0.25) (layer "B.Cu") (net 1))
 (segment (start 97.0548 43.4181) (end 97.4591 43.8224) (width 0.25) (layer "B.Cu") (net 1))
 (segment (start 93 35) (end 94.0767 35) (width 0.25) (layer "F.Cu") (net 9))
 (segment (start 94.0767 35.1347) (end 94.0767 35) (width 0.25) (layer "F.Cu") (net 9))
 (segment (start 97.875 38.095) (end 97.7185 38.095) (width 0.25) (layer "F.Cu") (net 9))
 (segment (start 95.744 36.1205) (end 95.0625 36.1205) (width 0.25) (layer "F.Cu") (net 9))
 (segment (start 97.7185 38.095) (end 95.744 36.1205) (width 0.25) (layer "F.Cu") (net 9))
 (segment (start 95.0625 36.1205) (end 94.0767 35.1347) (width 0.25) (layer "F.Cu") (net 9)))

